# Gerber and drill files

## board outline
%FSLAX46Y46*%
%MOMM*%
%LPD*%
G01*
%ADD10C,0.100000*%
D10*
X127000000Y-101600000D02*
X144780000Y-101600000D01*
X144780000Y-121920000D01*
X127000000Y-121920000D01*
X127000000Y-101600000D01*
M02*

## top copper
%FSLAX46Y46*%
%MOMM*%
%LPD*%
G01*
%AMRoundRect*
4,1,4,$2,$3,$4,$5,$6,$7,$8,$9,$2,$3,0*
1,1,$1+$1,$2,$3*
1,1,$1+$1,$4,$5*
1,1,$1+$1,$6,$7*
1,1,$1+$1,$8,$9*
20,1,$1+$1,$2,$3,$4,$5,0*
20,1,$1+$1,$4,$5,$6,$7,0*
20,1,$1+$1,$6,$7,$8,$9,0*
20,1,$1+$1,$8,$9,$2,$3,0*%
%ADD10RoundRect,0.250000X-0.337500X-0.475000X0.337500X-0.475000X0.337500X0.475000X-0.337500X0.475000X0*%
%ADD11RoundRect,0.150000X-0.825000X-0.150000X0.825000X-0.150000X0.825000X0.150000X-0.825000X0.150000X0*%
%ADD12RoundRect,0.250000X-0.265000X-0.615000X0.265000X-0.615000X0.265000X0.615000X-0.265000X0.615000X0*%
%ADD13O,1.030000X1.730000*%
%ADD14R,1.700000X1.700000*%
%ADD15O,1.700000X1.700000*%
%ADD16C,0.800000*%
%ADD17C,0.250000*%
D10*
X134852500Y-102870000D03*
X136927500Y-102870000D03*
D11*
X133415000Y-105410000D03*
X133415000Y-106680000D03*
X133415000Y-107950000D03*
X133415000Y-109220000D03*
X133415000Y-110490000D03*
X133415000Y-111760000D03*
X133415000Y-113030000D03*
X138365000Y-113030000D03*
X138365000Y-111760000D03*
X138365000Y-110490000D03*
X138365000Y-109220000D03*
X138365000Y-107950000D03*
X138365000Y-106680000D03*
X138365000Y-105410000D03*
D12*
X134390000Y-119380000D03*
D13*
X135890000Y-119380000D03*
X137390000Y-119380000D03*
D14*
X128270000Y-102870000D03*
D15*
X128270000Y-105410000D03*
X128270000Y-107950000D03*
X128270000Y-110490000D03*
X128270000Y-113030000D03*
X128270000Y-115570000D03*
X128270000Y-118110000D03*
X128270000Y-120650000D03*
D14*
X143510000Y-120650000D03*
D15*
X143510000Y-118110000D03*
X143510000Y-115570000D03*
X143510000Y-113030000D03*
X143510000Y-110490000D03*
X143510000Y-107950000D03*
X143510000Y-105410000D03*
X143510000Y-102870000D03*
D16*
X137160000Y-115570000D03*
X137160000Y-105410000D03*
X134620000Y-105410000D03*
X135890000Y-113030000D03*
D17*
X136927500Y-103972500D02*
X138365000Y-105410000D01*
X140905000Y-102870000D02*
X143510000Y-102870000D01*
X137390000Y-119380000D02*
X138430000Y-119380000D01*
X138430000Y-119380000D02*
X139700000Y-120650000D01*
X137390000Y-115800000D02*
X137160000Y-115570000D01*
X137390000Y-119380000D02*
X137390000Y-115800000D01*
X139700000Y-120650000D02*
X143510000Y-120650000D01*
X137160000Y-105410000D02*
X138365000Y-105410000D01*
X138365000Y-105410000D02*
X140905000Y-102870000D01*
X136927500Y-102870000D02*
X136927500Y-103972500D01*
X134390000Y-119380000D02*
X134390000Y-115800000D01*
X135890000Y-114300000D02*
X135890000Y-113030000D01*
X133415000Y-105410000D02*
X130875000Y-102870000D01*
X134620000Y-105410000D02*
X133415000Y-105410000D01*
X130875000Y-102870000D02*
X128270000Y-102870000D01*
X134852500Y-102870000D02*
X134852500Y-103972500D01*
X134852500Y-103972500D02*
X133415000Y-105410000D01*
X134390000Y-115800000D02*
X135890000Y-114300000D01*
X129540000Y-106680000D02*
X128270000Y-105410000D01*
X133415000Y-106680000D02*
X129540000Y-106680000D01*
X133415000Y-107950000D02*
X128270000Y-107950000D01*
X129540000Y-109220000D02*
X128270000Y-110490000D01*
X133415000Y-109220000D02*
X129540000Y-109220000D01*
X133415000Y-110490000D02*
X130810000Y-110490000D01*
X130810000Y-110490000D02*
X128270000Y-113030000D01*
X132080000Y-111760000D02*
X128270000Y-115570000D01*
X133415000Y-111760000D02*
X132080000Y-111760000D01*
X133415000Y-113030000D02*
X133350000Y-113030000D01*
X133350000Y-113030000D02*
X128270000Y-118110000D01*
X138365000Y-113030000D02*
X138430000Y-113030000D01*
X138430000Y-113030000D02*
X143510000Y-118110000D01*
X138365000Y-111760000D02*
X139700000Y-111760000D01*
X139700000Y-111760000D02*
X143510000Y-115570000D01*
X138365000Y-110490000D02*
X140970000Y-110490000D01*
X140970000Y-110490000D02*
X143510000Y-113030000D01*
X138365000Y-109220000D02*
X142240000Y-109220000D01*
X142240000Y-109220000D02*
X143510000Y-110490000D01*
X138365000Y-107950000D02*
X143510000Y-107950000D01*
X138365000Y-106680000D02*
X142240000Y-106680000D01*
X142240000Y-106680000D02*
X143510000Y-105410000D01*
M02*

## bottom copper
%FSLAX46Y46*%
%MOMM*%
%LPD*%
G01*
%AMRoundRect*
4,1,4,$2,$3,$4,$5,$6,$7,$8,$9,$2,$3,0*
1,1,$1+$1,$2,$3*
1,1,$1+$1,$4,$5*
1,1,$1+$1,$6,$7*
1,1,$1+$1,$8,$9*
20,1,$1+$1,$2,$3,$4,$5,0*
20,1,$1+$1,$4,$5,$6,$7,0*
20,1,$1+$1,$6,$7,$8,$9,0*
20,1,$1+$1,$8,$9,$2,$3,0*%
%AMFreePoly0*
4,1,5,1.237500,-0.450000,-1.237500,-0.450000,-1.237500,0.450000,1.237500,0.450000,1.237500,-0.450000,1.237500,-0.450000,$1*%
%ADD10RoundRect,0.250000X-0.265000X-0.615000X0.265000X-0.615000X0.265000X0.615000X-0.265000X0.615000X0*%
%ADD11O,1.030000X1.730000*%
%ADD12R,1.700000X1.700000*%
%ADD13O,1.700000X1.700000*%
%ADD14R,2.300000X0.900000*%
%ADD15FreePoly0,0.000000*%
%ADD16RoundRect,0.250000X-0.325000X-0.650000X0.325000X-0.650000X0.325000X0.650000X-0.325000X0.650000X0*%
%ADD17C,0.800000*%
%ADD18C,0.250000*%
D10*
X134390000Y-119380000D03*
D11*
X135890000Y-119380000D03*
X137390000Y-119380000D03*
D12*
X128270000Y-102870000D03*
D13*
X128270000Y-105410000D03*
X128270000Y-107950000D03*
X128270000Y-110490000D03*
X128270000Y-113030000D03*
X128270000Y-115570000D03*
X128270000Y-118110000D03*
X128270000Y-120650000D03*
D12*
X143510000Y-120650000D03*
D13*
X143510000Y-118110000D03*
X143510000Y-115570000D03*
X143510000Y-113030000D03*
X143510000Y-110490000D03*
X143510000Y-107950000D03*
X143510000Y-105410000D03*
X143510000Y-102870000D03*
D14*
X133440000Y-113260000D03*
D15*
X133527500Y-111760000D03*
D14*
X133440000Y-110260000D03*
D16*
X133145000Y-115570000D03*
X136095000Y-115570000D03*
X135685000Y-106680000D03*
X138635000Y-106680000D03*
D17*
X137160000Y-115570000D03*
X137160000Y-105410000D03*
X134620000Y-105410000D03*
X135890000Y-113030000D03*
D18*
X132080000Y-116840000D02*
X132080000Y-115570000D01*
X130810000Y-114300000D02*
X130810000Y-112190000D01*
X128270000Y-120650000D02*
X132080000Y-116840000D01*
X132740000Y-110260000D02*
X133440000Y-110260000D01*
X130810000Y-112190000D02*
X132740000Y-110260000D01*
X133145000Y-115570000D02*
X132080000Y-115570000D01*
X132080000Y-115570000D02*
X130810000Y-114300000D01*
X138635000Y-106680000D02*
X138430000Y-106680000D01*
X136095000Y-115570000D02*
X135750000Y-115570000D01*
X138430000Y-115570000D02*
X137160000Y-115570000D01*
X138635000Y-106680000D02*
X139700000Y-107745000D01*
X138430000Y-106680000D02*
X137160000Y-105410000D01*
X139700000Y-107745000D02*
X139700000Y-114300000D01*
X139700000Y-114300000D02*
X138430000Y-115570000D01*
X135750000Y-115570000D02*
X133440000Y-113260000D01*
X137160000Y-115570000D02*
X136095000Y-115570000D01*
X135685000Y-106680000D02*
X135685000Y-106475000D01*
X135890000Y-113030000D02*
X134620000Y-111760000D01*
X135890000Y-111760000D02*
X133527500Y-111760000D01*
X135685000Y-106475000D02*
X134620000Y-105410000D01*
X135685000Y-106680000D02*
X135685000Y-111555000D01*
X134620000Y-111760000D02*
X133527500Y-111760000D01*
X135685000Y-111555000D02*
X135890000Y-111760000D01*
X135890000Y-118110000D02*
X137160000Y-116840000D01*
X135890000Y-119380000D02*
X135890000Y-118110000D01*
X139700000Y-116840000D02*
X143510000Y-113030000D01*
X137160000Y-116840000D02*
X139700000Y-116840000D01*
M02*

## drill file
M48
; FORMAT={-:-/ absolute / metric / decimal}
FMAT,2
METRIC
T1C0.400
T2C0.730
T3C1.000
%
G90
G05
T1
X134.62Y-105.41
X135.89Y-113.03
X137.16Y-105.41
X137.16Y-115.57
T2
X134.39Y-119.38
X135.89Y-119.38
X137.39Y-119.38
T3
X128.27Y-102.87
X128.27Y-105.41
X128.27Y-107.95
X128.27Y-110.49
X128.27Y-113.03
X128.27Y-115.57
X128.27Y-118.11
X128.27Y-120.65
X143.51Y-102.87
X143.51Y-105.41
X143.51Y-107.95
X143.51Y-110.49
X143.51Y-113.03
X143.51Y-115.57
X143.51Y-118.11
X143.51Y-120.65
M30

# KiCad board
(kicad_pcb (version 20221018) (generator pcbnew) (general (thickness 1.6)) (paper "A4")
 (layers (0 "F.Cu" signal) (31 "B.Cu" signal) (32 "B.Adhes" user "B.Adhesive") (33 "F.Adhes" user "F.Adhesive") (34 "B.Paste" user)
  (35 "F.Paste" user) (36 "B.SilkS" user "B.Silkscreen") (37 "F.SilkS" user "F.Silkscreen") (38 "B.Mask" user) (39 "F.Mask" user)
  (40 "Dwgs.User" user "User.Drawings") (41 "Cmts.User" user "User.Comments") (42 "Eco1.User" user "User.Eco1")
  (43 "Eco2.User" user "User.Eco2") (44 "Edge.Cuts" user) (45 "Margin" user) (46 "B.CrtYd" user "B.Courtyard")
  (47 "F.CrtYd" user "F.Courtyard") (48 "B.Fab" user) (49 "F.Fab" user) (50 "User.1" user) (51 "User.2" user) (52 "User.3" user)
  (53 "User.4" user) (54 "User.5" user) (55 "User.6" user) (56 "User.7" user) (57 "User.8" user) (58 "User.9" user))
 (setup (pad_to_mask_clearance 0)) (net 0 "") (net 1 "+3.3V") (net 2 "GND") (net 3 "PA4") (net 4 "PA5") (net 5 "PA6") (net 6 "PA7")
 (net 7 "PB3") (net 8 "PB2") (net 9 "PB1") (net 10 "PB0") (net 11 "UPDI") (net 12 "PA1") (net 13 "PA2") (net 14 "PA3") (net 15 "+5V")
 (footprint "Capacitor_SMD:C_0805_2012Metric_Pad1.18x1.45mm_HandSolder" (layer "F.Cu") (at 135.89 102.87)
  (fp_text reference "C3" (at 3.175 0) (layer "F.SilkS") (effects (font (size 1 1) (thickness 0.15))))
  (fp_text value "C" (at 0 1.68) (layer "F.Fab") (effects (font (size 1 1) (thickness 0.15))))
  (pad "1" smd roundrect (at -1.0375 0) (size 1.175 1.45) (layers "F.Cu" "F.Paste" "F.Mask") (roundrect_rratio 0.2127659574) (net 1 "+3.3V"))
  (pad "2" smd roundrect (at 1.0375 0) (size 1.175 1.45) (layers "F.Cu" "F.Paste" "F.Mask") (roundrect_rratio 0.2127659574) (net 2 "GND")))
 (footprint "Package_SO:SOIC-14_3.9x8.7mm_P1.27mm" (layer "F.Cu") (at 135.89 109.22)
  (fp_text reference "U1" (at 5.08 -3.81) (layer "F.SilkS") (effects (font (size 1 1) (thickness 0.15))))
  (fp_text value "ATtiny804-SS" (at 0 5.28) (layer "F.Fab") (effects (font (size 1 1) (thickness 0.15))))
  (pad "1" smd roundrect (at -2.475 -3.81) (size 1.95 0.6) (layers "F.Cu" "F.Paste" "F.Mask") (roundrect_rratio 0.25) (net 1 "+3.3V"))
  (pad "2" smd roundrect (at -2.475 -2.54) (size 1.95 0.6) (layers "F.Cu" "F.Paste" "F.Mask") (roundrect_rratio 0.25) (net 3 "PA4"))
  (pad "3" smd roundrect (at -2.475 -1.27) (size 1.95 0.6) (layers "F.Cu" "F.Paste" "F.Mask") (roundrect_rratio 0.25) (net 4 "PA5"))
  (pad "4" smd roundrect (at -2.475 0) (size 1.95 0.6) (layers "F.Cu" "F.Paste" "F.Mask") (roundrect_rratio 0.25) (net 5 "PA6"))
  (pad "5" smd roundrect (at -2.475 1.27) (size 1.95 0.6) (layers "F.Cu" "F.Paste" "F.Mask") (roundrect_rratio 0.25) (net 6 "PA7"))
  (pad "6" smd roundrect (at -2.475 2.54) (size 1.95 0.6) (layers "F.Cu" "F.Paste" "F.Mask") (roundrect_rratio 0.25) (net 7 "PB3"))
  (pad "7" smd roundrect (at -2.475 3.81) (size 1.95 0.6) (layers "F.Cu" "F.Paste" "F.Mask") (roundrect_rratio 0.25) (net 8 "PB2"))
  (pad "8" smd roundrect (at 2.475 3.81) (size 1.95 0.6) (layers "F.Cu" "F.Paste" "F.Mask") (roundrect_rratio 0.25) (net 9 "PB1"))
  (pad "9" smd roundrect (at 2.475 2.54) (size 1.95 0.6) (layers "F.Cu" "F.Paste" "F.Mask") (roundrect_rratio 0.25) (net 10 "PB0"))
  (pad "10" smd roundrect (at 2.475 1.27) (size 1.95 0.6) (layers "F.Cu" "F.Paste" "F.Mask") (roundrect_rratio 0.25) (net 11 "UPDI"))
  (pad "11" smd roundrect (at 2.475 0) (size 1.95 0.6) (layers "F.Cu" "F.Paste" "F.Mask") (roundrect_rratio 0.25) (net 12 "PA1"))
  (pad "12" smd roundrect (at 2.475 -1.27) (size 1.95 0.6) (layers "F.Cu" "F.Paste" "F.Mask") (roundrect_rratio 0.25) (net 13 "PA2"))
  (pad "13" smd roundrect (at 2.475 -2.54) (size 1.95 0.6) (layers "F.Cu" "F.Paste" "F.Mask") (roundrect_rratio 0.25) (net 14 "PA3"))
  (pad "14" smd roundrect (at 2.475 -3.81) (size 1.95 0.6) (layers "F.Cu" "F.Paste" "F.Mask") (roundrect_rratio 0.25) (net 2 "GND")))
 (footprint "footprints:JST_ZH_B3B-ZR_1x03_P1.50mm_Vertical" (layer "F.Cu") (at 134.39 119.38)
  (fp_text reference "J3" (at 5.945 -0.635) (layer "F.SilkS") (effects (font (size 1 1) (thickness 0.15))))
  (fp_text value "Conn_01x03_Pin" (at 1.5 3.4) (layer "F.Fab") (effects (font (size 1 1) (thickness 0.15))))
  (pad "1" thru_hole roundrect (at 0 0) (size 1.03 1.73) (drill 0.73) (layers "*.Cu" "*.Mask") (roundrect_rratio 0.2427184466)
   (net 1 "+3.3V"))
  (pad "2" thru_hole oval (at 1.5 0) (size 1.03 1.73) (drill 0.73) (layers "*.Cu" "*.Mask") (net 11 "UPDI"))
  (pad "3" thru_hole oval (at 3 0) (size 1.03 1.73) (drill 0.73) (layers "*.Cu" "*.Mask") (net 2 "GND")))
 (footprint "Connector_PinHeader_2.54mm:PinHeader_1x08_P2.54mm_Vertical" (layer "F.Cu") (at 128.27 102.87)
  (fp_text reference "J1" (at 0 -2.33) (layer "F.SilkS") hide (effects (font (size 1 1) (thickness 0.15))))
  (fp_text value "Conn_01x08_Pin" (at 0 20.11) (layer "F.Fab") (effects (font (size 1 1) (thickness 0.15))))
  (pad "1" thru_hole rect (at 0 0) (size 1.7 1.7) (drill 1) (layers "*.Cu" "*.Mask") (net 1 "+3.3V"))
  (pad "2" thru_hole oval (at 0 2.54) (size 1.7 1.7) (drill 1) (layers "*.Cu" "*.Mask") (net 3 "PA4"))
  (pad "3" thru_hole oval (at 0 5.08) (size 1.7 1.7) (drill 1) (layers "*.Cu" "*.Mask") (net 4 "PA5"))
  (pad "4" thru_hole oval (at 0 7.62) (size 1.7 1.7) (drill 1) (layers "*.Cu" "*.Mask") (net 5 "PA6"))
  (pad "5" thru_hole oval (at 0 10.16) (size 1.7 1.7) (drill 1) (layers "*.Cu" "*.Mask") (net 6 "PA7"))
  (pad "6" thru_hole oval (at 0 12.7) (size 1.7 1.7) (drill 1) (layers "*.Cu" "*.Mask") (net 7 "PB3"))
  (pad "7" thru_hole oval (at 0 15.24) (size 1.7 1.7) (drill 1) (layers "*.Cu" "*.Mask") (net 8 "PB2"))
  (pad "8" thru_hole oval (at 0 17.78) (size 1.7 1.7) (drill 1) (layers "*.Cu" "*.Mask") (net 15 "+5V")))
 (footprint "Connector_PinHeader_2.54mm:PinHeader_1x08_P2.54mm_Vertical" (layer "F.Cu") (at 143.51 120.65 180)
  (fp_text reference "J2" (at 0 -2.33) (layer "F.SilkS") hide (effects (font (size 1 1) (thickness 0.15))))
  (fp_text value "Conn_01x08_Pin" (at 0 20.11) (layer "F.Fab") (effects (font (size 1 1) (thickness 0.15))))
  (pad "1" thru_hole rect (at 0 0 180) (size 1.7 1.7) (drill 1) (layers "*.Cu" "*.Mask") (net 2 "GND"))
  (pad "2" thru_hole oval (at 0 2.54 180) (size 1.7 1.7) (drill 1) (layers "*.Cu" "*.Mask") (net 9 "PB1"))
  (pad "3" thru_hole oval (at 0 5.08 180) (size 1.7 1.7) (drill 1) (layers "*.Cu" "*.Mask") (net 10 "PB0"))
  (pad "4" thru_hole oval (at 0 7.62 180) (size 1.7 1.7) (drill 1) (layers "*.Cu" "*.Mask") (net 11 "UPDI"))
  (pad "5" thru_hole oval (at 0 10.16 180) (size 1.7 1.7) (drill 1) (layers "*.Cu" "*.Mask") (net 12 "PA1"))
  (pad "6" thru_hole oval (at 0 12.7 180) (size 1.7 1.7) (drill 1) (layers "*.Cu" "*.Mask") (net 13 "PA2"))
  (pad "7" thru_hole oval (at 0 15.24 180) (size 1.7 1.7) (drill 1) (layers "*.Cu" "*.Mask") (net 14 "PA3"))
  (pad "8" thru_hole oval (at 0 17.78 180) (size 1.7 1.7) (drill 1) (layers "*.Cu" "*.Mask") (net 2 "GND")))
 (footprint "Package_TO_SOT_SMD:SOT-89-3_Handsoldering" (layer "B.Cu") (at 135.89 111.76)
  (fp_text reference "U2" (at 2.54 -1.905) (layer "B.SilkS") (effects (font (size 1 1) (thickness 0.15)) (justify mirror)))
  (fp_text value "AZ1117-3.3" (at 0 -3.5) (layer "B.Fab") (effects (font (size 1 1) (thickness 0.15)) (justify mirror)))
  (pad "1" smd rect (at -2.45 1.5) (size 2.3 0.9) (layers "B.Cu" "B.Paste" "B.Mask") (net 2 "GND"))
  (pad "2" smd custom (at -2.3625 0) (size 2.475 0.9) (layers "B.Cu" "B.Paste" "B.Mask") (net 1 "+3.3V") (zone_connect 2)
   (thermal_bridge_angle 45) (options (clearance outline) (anchor rect)) (primitives))
  (pad "3" smd rect (at -2.45 -1.5) (size 2.3 0.9) (layers "B.Cu" "B.Paste" "B.Mask") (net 15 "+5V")))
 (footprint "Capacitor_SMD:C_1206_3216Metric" (layer "B.Cu") (at 134.62 115.57)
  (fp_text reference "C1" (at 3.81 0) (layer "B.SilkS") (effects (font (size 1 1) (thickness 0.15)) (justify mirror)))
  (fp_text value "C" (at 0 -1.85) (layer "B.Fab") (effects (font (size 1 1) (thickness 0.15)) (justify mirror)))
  (pad "1" smd roundrect (at -1.475 0) (size 1.15 1.8) (layers "B.Cu" "B.Paste" "B.Mask") (roundrect_rratio 0.2173913043) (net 15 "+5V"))
  (pad "2" smd roundrect (at 1.475 0) (size 1.15 1.8) (layers "B.Cu" "B.Paste" "B.Mask") (roundrect_rratio 0.2173913043) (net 2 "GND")))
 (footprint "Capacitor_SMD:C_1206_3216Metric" (layer "B.Cu") (at 137.16 106.68)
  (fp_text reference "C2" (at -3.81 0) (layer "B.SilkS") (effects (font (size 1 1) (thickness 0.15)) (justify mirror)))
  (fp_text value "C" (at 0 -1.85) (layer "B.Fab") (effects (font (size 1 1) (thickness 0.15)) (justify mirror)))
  (pad "1" smd roundrect (at -1.475 0) (size 1.15 1.8) (layers "B.Cu" "B.Paste" "B.Mask") (roundrect_rratio 0.2173913043) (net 1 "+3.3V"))
  (pad "2" smd roundrect (at 1.475 0) (size 1.15 1.8) (layers "B.Cu" "B.Paste" "B.Mask") (roundrect_rratio 0.2173913043) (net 2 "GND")))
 (gr_rect (start 127 101.6) (end 144.78 121.92) (stroke (width 0.1) (type default)) (fill none) (layer "Edge.Cuts"))
 (segment (start 132.08 116.84) (end 132.08 115.57) (width 0.25) (layer "B.Cu") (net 15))
 (segment (start 130.81 114.3) (end 130.81 112.19) (width 0.25) (layer "B.Cu") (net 15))
 (segment (start 128.27 120.65) (end 132.08 116.84) (width 0.25) (layer "B.Cu") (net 15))
 (segment (start 132.74 110.26) (end 133.44 110.26) (width 0.25) (layer "B.Cu") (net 15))
 (segment (start 130.81 112.19) (end 132.74 110.26) (width 0.25) (layer "B.Cu") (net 15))
 (segment (start 133.145 115.57) (end 132.08 115.57) (width 0.25) (layer "B.Cu") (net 15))
 (segment (start 132.08 115.57) (end 130.81 114.3) (width 0.25) (layer "B.Cu") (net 15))
 (segment (start 136.9275 103.9725) (end 138.365 105.41) (width 0.25) (layer "F.Cu") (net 2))
 (segment (start 140.905 102.87) (end 143.51 102.87) (width 0.25) (layer "F.Cu") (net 2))
 (segment (start 137.39 119.38) (end 138.43 119.38) (width 0.25) (layer "F.Cu") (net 2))
 (segment (start 138.43 119.38) (end 139.7 120.65) (width 0.25) (layer "F.Cu") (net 2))
 (segment (start 137.39 115.8) (end 137.16 115.57) (width 0.25) (layer "F.Cu") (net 2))
 (segment (start 137.39 119.38) (end 137.39 115.8) (width 0.25) (layer "F.Cu") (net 2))
 (segment (start 139.7 120.65) (end 143.51 120.65) (width 0.25) (layer "F.Cu") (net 2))
 (segment (start 137.16 105.41) (end 138.365 105.41) (width 0.25) (layer "F.Cu") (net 2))
 (segment (start 138.365 105.41) (end 140.905 102.87) (width 0.25) (layer "F.Cu") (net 2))
 (segment (start 136.9275 102.87) (end 136.9275 103.9725) (width 0.25) (layer "F.Cu") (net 2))
 (via (at 137.16 115.57) (size 0.8) (drill 0.4) (layers "F.Cu" "B.Cu") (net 2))
 (via (at 137.16 105.41) (size 0.8) (drill 0.4) (layers "F.Cu" "B.Cu") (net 2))
 (segment (start 138.635 106.68) (end 138.43 106.68) (width 0.25) (layer "B.Cu") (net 2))
 (segment (start 136.095 115.57) (end 135.75 115.57) (width 0.25) (layer "B.Cu") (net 2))
 (segment (start 138.43 115.57) (end 137.16 115.57) (width 0.25) (layer "B.Cu") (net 2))
 (segment (start 138.635 106.68) (end 139.7 107.745) (width 0.25) (layer "B.Cu") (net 2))
 (segment (start 138.43 106.68) (end 137.16 105.41) (width 0.25) (layer "B.Cu") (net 2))
 (segment (start 139.7 107.745) (end 139.7 114.3) (width 0.25) (layer "B.Cu") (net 2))
 (segment (start 139.7 114.3) (end 138.43 115.57) (width 0.25) (layer "B.Cu") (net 2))
 (segment (start 135.75 115.57) (end 133.44 113.26) (width 0.25) (layer "B.Cu") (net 2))
 (segment (start 137.16 115.57) (end 136.095 115.57) (width 0.25) (layer "B.Cu") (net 2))
 (segment (start 134.39 119.38) (end 134.39 115.8) (width 0.25) (layer "F.Cu") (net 1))
 (segment (start 135.89 114.3) (end 135.89 113.03) (width 0.25) (layer "F.Cu") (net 1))
 (segment (start 133.415 105.41) (end 130.875 102.87) (width 0.25) (layer "F.Cu") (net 1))
 (segment (start 134.62 105.41) (end 133.415 105.41) (width 0.25) (layer "F.Cu") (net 1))
 (segment (start 130.875 102.87) (end 128.27 102.87) (width 0.25) (layer "F.Cu") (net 1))
 (segment (start 134.8525 102.87) (end 134.8525 103.9725) (width 0.25) (layer "F.Cu") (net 1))
 (segment (start 134.8525 103.9725) (end 133.415 105.41) (width 0.25) (layer "F.Cu") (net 1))
 (segment (start 134.39 115.8) (end 135.89 114.3) (width 0.25) (layer "F.Cu") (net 1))
 (via (at 134.62 105.41) (size 0.8) (drill 0.4) (layers "F.Cu" "B.Cu") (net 1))
 (via (at 135.89 113.03) (size 0.8) (drill 0.4) (layers "F.Cu" "B.Cu") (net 1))
 (segment (start 135.685 106.68) (end 135.685 106.475) (width 0.25) (layer "B.Cu") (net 1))
 (segment (start 135.89 113.03) (end 134.62 111.76) (width 0.25) (layer "B.Cu") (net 1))
 (segment (start 135.89 111.76) (end 133.5275 111.76) (width 0.25) (layer "B.Cu") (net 1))
 (segment (start 135.685 106.475) (end 134.62 105.41) (width 0.25) (layer "B.Cu") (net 1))
 (segment (start 135.685 106.68) (end 135.685 111.555) (width 0.25) (layer "B.Cu") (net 1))
 (segment (start 134.62 111.76) (end 133.5275 111.76) (width 0.25) (layer "B.Cu") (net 1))
 (segment (start 135.685 111.555) (end 135.89 111.76) (width 0.25) (layer "B.Cu") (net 1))
 (segment (start 129.54 106.68) (end 128.27 105.41) (width 0.25) (layer "F.Cu") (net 3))
 (segment (start 133.415 106.68) (end 129.54 106.68) (width 0.25) (layer "F.Cu") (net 3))
 (segment (start 133.415 107.95) (end 128.27 107.95) (width 0.25) (layer "F.Cu") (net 4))
 (segment (start 129.54 109.22) (end 128.27 110.49) (width 0.25) (layer "F.Cu") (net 5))
 (segment (start 133.415 109.22) (end 129.54 109.22) (width 0.25) (layer "F.Cu") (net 5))
 (segment (start 133.415 110.49) (end 130.81 110.49) (width 0.25) (layer "F.Cu") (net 6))
 (segment (start 130.81 110.49) (end 128.27 113.03) (width 0.25) (layer "F.Cu") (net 6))
 (segment (start 132.08 111.76) (end 128.27 115.57) (width 0.25) (layer "F.Cu") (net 7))
 (segment (start 133.415 111.76) (end 132.08 111.76) (width 0.25) (layer "F.Cu") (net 7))
 (segment (start 133.415 113.03) (end 133.35 113.03) (width 0.25) (layer "F.Cu") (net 8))
 (segment (start 133.35 113.03) (end 128.27 118.11) (width 0.25) (layer "F.Cu") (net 8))
 (segment (start 138.365 113.03) (end 138.43 113.03) (width 0.25) (layer "F.Cu") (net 9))
 (segment (start 138.43 113.03) (end 143.51 118.11) (width 0.25) (layer "F.Cu") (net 9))
 (segment (start 138.365 111.76) (end 139.7 111.76) (width 0.25) (layer "F.Cu") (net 10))
 (segment (start 139.7 111.76) (end 143.51 115.57) (width 0.25) (layer "F.Cu") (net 10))
 (segment (start 138.365 110.49) (end 140.97 110.49) (width 0.25) (layer "F.Cu") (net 11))
 (segment (start 140.97 110.49) (end 143.51 113.03) (width 0.25) (layer "F.Cu") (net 11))
 (segment (start 135.89 118.11) (end 137.16 116.84) (width 0.25) (layer "B.Cu") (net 11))
 (segment (start 135.89 119.38) (end 135.89 118.11) (width 0.25) (layer "B.Cu") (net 11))
 (segment (start 139.7 116.84) (end 143.51 113.03) (width 0.25) (layer "B.Cu") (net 11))
 (segment (start 137.16 116.84) (end 139.7 116.84) (width 0.25) (layer "B.Cu") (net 11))
 (segment (start 138.365 109.22) (end 142.24 109.22) (width 0.25) (layer "F.Cu") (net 12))
 (segment (start 142.24 109.22) (end 143.51 110.49) (width 0.25) (layer "F.Cu") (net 12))
 (segment (start 138.365 107.95) (end 143.51 107.95) (width 0.25) (layer "F.Cu") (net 13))
 (segment (start 138.365 106.68) (end 142.24 106.68) (width 0.25) (layer "F.Cu") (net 14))
 (segment (start 142.24 106.68) (end 143.51 105.41) (width 0.25) (layer "F.Cu") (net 14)))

